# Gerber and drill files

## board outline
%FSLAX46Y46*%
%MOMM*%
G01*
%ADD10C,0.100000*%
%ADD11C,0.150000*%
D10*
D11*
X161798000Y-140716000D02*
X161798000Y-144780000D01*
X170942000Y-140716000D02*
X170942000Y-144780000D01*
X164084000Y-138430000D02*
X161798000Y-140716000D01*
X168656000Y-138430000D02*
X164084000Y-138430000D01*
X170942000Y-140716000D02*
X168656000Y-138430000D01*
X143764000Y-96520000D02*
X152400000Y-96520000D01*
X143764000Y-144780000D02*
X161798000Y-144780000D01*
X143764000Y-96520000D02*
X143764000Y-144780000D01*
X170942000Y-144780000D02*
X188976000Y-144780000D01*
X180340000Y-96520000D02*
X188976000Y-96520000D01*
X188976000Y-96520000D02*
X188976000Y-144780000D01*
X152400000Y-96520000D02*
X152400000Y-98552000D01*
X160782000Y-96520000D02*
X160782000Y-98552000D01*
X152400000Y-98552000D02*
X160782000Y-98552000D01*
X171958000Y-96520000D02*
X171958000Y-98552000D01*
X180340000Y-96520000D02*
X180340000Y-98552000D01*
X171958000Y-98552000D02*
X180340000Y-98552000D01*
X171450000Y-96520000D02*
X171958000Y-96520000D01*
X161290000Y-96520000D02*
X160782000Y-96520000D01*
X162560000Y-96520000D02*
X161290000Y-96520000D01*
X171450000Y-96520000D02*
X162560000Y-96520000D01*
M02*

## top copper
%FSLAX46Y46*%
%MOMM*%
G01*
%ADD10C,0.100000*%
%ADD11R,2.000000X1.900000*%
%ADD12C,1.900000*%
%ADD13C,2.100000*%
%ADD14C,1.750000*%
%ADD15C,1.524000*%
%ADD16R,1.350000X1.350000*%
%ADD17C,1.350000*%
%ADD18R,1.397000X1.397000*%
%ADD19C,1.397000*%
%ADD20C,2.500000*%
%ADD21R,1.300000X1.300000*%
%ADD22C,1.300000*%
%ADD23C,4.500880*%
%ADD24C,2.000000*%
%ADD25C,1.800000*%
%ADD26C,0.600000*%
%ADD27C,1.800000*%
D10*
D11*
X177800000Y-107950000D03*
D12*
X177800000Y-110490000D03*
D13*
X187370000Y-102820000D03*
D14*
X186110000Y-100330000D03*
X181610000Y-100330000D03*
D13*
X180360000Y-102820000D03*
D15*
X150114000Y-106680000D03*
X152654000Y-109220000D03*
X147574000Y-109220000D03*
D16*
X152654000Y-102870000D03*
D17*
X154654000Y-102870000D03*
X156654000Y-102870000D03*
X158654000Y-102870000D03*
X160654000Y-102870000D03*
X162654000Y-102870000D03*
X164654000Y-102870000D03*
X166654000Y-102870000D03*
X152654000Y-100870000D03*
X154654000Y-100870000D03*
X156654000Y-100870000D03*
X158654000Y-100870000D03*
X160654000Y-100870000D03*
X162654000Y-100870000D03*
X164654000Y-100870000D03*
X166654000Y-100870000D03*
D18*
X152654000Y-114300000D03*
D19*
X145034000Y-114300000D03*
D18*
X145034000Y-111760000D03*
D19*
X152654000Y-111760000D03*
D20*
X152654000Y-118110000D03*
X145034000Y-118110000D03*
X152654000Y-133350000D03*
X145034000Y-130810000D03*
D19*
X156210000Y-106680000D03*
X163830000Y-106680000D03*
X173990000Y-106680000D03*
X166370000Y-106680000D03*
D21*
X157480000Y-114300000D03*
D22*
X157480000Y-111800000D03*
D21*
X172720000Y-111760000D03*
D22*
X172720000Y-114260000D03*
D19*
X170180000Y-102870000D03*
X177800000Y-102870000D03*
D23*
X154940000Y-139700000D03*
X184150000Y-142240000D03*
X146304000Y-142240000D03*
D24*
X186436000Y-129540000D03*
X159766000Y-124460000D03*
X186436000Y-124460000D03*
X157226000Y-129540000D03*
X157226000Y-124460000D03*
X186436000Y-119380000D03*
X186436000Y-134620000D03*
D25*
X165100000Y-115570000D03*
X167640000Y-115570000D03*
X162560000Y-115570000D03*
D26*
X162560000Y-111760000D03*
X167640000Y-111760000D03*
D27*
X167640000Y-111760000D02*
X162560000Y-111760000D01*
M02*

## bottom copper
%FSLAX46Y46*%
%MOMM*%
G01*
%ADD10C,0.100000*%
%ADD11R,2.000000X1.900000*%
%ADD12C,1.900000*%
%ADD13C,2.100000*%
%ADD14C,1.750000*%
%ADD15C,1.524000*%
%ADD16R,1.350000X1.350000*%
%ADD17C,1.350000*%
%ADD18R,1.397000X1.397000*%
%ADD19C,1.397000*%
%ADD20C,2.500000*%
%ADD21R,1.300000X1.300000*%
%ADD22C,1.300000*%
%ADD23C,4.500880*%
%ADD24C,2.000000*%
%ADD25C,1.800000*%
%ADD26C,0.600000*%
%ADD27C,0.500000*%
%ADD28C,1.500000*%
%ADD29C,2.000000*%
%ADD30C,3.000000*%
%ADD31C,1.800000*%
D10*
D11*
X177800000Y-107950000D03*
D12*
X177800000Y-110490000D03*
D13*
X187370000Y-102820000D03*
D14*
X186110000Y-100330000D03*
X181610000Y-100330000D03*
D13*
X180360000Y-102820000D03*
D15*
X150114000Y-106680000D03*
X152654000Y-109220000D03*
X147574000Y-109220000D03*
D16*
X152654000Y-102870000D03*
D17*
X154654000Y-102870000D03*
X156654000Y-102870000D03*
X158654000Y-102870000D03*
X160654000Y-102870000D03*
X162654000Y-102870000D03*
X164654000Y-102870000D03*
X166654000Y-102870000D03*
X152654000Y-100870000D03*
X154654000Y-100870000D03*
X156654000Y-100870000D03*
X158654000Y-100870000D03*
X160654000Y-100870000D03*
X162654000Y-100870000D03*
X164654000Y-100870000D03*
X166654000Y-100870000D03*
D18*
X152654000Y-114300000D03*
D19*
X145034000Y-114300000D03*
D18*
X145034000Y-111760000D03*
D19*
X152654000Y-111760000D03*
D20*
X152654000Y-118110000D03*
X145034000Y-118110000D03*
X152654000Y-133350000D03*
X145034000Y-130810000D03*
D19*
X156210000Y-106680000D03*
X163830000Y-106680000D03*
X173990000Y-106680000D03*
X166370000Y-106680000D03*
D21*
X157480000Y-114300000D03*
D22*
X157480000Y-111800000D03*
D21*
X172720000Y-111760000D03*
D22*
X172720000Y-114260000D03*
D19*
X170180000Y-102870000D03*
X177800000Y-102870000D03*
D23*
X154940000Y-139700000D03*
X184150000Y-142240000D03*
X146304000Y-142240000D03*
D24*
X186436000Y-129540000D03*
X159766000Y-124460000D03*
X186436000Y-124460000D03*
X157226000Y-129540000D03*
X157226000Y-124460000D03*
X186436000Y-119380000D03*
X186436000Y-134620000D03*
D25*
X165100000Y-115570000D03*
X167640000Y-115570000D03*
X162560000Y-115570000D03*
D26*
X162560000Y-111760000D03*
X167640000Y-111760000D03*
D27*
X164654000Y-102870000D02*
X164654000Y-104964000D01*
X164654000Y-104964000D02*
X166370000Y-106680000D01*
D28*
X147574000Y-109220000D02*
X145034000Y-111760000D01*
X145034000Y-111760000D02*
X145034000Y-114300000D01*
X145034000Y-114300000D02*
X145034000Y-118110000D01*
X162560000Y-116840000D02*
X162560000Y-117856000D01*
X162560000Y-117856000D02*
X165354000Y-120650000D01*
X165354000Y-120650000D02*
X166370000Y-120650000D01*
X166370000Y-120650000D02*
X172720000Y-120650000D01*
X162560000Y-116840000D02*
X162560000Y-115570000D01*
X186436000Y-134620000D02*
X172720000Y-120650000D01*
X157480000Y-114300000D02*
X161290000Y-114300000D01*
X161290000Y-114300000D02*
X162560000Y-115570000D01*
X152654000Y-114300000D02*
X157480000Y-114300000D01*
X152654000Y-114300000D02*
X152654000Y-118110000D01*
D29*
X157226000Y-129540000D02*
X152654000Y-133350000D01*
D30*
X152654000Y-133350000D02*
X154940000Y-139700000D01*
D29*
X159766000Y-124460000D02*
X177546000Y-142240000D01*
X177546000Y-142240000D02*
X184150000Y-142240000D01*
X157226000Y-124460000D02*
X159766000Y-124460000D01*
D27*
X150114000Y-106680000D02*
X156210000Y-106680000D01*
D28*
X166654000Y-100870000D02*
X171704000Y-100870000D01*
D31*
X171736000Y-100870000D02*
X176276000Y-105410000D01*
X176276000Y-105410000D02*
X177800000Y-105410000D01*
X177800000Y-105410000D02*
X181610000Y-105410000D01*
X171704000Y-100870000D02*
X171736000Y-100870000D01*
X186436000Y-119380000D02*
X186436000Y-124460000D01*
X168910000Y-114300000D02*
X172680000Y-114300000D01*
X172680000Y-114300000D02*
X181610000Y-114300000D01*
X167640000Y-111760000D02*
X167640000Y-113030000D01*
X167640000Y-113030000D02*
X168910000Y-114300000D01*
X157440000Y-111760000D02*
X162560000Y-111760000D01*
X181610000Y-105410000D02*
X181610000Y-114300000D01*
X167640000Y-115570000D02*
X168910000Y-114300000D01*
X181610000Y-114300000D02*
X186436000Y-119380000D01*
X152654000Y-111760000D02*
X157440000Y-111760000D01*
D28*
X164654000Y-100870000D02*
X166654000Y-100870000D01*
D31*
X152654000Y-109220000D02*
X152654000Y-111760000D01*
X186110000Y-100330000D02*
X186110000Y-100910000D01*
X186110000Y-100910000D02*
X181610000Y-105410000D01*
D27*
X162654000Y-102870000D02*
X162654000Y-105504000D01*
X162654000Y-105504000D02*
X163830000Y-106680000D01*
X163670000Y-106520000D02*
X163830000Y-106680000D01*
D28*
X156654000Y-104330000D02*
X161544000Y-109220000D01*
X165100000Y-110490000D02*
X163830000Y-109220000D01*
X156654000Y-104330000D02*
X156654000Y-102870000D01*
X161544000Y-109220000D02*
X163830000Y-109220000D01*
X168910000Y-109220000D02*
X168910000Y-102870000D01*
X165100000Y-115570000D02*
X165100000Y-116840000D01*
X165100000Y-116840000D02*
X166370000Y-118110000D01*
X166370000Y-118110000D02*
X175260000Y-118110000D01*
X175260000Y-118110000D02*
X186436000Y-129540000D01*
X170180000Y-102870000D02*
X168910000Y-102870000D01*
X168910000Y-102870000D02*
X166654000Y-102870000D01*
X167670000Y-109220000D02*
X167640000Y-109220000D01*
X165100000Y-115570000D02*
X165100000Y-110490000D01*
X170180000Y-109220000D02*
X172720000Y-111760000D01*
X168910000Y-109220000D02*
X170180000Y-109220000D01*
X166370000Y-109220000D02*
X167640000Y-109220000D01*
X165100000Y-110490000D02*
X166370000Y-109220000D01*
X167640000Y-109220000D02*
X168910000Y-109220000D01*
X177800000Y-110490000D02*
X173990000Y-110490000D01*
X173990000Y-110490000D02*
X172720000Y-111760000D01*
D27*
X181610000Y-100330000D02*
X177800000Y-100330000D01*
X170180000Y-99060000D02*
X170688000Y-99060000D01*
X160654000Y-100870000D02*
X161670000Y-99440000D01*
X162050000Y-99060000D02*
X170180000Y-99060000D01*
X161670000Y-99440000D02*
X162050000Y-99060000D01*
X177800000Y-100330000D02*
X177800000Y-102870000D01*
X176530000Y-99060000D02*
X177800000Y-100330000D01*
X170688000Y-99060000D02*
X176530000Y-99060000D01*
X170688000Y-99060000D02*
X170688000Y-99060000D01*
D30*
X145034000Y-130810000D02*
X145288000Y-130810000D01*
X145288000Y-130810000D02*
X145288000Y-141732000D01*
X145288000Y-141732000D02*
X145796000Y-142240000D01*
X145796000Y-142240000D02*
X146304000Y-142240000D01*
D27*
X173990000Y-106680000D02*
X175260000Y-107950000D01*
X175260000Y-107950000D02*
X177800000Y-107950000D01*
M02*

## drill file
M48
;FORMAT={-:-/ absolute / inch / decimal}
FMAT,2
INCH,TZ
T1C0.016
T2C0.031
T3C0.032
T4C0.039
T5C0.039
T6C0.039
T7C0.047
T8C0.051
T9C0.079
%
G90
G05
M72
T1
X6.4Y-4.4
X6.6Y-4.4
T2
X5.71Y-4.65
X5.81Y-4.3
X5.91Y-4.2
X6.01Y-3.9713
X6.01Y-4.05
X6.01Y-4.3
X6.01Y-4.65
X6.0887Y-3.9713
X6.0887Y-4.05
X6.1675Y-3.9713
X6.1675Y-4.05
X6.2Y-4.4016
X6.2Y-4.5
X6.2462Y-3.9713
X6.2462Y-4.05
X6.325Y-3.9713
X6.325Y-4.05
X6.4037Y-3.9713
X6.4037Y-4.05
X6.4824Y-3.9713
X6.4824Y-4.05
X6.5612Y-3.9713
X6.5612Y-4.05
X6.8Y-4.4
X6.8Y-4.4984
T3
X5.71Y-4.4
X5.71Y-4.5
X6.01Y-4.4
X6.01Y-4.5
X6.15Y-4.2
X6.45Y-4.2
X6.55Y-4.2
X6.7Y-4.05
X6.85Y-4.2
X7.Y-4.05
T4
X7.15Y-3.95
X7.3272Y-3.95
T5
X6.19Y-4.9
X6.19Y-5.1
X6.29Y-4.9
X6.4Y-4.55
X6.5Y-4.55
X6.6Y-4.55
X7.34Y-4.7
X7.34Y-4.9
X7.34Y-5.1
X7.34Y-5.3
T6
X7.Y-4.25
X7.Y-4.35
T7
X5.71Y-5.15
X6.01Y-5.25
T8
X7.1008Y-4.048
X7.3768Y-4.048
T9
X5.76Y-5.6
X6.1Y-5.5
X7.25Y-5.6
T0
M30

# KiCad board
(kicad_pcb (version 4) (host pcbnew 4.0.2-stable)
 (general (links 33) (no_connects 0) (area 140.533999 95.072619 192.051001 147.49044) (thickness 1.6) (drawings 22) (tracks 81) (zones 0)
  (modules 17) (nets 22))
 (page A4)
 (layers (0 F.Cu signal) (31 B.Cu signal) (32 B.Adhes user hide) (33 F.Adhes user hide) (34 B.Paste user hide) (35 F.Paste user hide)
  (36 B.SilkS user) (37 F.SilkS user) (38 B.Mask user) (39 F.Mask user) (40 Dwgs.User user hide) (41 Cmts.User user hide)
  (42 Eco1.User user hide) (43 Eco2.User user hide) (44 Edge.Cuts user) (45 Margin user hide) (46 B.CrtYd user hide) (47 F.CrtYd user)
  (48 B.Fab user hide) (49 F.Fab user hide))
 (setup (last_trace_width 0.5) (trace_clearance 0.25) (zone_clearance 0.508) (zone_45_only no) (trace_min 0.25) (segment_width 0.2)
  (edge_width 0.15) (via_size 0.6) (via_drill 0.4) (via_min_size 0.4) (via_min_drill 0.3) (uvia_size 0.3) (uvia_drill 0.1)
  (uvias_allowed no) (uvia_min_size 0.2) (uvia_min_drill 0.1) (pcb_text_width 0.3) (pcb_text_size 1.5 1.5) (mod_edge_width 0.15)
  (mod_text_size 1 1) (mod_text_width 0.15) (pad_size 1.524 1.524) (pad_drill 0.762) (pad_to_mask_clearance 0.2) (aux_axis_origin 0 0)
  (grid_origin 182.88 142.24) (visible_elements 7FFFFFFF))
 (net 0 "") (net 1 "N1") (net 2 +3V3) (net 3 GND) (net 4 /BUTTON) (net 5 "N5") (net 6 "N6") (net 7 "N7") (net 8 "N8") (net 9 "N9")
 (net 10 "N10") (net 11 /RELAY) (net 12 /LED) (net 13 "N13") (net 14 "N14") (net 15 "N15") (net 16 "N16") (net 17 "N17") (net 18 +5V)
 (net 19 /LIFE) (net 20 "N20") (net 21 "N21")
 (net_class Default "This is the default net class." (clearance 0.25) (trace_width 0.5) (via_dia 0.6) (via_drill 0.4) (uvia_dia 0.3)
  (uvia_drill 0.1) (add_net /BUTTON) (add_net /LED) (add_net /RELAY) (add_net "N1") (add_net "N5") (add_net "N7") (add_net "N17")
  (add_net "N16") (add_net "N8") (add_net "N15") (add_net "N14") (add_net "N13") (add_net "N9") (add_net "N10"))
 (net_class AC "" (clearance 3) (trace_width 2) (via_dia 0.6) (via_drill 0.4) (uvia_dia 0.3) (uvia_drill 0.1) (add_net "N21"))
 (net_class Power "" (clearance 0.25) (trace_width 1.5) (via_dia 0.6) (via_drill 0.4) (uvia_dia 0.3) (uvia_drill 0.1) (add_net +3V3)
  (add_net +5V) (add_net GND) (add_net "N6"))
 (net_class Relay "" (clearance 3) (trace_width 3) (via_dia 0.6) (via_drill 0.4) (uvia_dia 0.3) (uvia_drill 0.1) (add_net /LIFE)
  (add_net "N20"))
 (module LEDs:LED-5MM (layer F.Cu) (at 177.8 107.95 270)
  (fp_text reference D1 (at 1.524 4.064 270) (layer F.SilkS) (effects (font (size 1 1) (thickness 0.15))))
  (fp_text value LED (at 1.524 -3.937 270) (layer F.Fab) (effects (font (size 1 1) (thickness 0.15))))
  (pad 1 thru_hole rect (at 0 0) (size 2 1.9) (drill 1.00076) (layers *.Cu *.Mask F.SilkS) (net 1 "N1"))
  (pad 2 thru_hole circle (at 2.54 0 270) (size 1.9 1.9) (drill 1.00076) (layers *.Cu *.Mask F.SilkS) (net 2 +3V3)))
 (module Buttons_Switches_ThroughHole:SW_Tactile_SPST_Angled (layer F.Cu) (at 181.61 100.33)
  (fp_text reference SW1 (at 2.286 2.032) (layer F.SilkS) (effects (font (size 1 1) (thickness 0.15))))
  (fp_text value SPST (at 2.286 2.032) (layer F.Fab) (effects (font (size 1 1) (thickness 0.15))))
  (pad "" thru_hole circle (at 5.76 2.49) (size 2.1 2.1) (drill 1.3) (layers *.Cu *.Mask F.SilkS))
  (pad 2 thru_hole circle (at 4.5 0) (size 1.75 1.75) (drill 0.99) (layers *.Cu *.Mask F.SilkS) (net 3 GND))
  (pad 1 thru_hole circle (at 0 0) (size 1.75 1.75) (drill 0.99) (layers *.Cu *.Mask F.SilkS) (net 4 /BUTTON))
  (pad "" thru_hole circle (at -1.25 2.49) (size 2.1 2.1) (drill 1.3) (layers *.Cu *.Mask F.SilkS)))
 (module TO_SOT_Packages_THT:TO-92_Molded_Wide (layer F.Cu) (at 147.574 109.22)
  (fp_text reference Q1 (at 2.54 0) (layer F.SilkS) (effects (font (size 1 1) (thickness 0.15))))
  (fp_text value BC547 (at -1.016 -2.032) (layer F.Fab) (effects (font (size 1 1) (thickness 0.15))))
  (pad 2 thru_hole circle (at 2.54 -2.54 90) (size 1.524 1.524) (drill 0.8) (layers *.Cu *.Mask F.SilkS) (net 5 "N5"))
  (pad 3 thru_hole circle (at 5.08 0 90) (size 1.524 1.524) (drill 0.8) (layers *.Cu *.Mask F.SilkS) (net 3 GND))
  (pad 1 thru_hole circle (at 0 0 90) (size 1.524 1.524) (drill 0.8) (layers *.Cu *.Mask F.SilkS) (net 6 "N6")))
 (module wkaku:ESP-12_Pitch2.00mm (layer F.Cu) (at 152.654 102.87 90)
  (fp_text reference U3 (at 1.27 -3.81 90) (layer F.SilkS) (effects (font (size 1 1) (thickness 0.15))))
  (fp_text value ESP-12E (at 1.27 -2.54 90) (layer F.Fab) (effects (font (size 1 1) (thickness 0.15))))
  (pad 1 thru_hole rect (at 0 0 90) (size 1.35 1.35) (drill 0.8) (layers *.Cu *.Mask) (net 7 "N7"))
  (pad 2 thru_hole circle (at 0 2 90) (size 1.35 1.35) (drill 0.8) (layers *.Cu *.Mask) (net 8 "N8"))
  (pad 3 thru_hole circle (at 0 4 90) (size 1.35 1.35) (drill 0.8) (layers *.Cu *.Mask) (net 2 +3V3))
  (pad 4 thru_hole circle (at 0 6 90) (size 1.35 1.35) (drill 0.8) (layers *.Cu *.Mask) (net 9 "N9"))
  (pad 5 thru_hole circle (at 0 8 90) (size 1.35 1.35) (drill 0.8) (layers *.Cu *.Mask) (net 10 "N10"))
  (pad 6 thru_hole circle (at 0 10 90) (size 1.35 1.35) (drill 0.8) (layers *.Cu *.Mask) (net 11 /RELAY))
  (pad 7 thru_hole circle (at 0 12 90) (size 1.35 1.35) (drill 0.8) (layers *.Cu *.Mask) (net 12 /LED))
  (pad 8 thru_hole circle (at 0 14 90) (size 1.35 1.35) (drill 0.8) (layers *.Cu *.Mask) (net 2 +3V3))
  (pad 22 thru_hole circle (at 2 0 90) (size 1.35 1.35) (drill 0.8) (layers *.Cu *.Mask) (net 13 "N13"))
  (pad 21 thru_hole circle (at 2 2 90) (size 1.35 1.35) (drill 0.8) (layers *.Cu *.Mask) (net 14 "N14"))
  (pad 20 thru_hole circle (at 2 4 90) (size 1.35 1.35) (drill 0.8) (layers *.Cu *.Mask) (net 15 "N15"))
  (pad 19 thru_hole circle (at 2 6 90) (size 1.35 1.35) (drill 0.8) (layers *.Cu *.Mask) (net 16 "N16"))
  (pad 18 thru_hole circle (at 2 8 90) (size 1.35 1.35) (drill 0.8) (layers *.Cu *.Mask) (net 4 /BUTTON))
  (pad 17 thru_hole circle (at 2 10 90) (size 1.35 1.35) (drill 0.8) (layers *.Cu *.Mask) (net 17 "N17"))
  (pad 16 thru_hole circle (at 2 12 90) (size 1.35 1.35) (drill 0.8) (layers *.Cu *.Mask) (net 3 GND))
  (pad 15 thru_hole circle (at 2 14 90) (size 1.35 1.35) (drill 0.8) (layers *.Cu *.Mask) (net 3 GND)))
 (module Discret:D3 (layer F.Cu) (at 148.844 114.3)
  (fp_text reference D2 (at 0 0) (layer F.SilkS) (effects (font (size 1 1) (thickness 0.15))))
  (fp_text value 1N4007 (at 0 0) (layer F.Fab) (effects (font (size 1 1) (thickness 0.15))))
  (pad 1 thru_hole rect (at 3.81 0) (size 1.397 1.397) (drill 0.8128) (layers *.Cu *.Mask F.SilkS) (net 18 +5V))
  (pad 2 thru_hole circle (at -3.81 0) (size 1.397 1.397) (drill 0.8128) (layers *.Cu *.Mask F.SilkS) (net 6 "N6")))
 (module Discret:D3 (layer F.Cu) (at 148.844 111.76 180)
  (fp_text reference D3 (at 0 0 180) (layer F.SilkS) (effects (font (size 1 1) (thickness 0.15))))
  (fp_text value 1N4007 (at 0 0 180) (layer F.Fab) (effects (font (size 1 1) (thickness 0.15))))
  (pad 1 thru_hole rect (at 3.81 0 180) (size 1.397 1.397) (drill 0.8128) (layers *.Cu *.Mask F.SilkS) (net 6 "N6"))
  (pad 2 thru_hole circle (at -3.81 0 180) (size 1.397 1.397) (drill 0.8128) (layers *.Cu *.Mask F.SilkS) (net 3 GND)))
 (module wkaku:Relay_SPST (layer F.Cu) (at 145.034 118.11 270)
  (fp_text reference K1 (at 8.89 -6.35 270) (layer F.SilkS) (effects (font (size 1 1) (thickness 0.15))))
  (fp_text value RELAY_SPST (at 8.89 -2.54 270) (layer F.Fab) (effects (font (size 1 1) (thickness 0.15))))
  (pad A1 thru_hole circle (at 0 -7.62 270) (size 2.5 2.5) (drill 0.8) (layers *.Cu *.Mask F.SilkS) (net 18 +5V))
  (pad A2 thru_hole circle (at 0 0 270) (size 2.5 2.5) (drill 0.8) (layers *.Cu *.Mask F.SilkS) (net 6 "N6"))
  (pad 7 thru_hole circle (at 15.24 -7.62 270) (size 2.5 2.5) (drill 1.19888) (layers *.Cu *.Mask F.SilkS) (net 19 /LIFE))
  (pad 5 thru_hole circle (at 12.7 0 270) (size 2.5 2.5) (drill 1.19888) (layers *.Cu *.Mask F.SilkS) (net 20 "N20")))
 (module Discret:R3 (layer F.Cu) (at 160.02 106.68)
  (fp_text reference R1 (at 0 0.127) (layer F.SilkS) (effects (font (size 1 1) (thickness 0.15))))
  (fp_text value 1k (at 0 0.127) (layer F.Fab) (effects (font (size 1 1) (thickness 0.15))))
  (pad 1 thru_hole circle (at -3.81 0) (size 1.397 1.397) (drill 0.8128) (layers *.Cu *.Mask F.SilkS) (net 5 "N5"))
  (pad 2 thru_hole circle (at 3.81 0) (size 1.397 1.397) (drill 0.8128) (layers *.Cu *.Mask F.SilkS) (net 11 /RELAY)))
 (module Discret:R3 (layer F.Cu) (at 170.18 106.68 180)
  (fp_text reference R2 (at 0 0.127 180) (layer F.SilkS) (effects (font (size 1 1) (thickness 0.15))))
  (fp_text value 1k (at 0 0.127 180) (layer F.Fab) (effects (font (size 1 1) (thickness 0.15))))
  (pad 1 thru_hole circle (at -3.81 0 180) (size 1.397 1.397) (drill 0.8128) (layers *.Cu *.Mask F.SilkS) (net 1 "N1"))
  (pad 2 thru_hole circle (at 3.81 0 180) (size 1.397 1.397) (drill 0.8128) (layers *.Cu *.Mask F.SilkS) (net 12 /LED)))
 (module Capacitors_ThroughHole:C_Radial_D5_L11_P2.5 (layer F.Cu) (at 157.48 114.3 90)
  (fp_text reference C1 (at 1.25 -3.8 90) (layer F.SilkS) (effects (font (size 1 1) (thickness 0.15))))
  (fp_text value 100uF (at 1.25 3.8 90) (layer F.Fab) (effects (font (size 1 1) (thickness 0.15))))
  (pad 1 thru_hole rect (at 0 0 90) (size 1.3 1.3) (drill 0.8) (layers *.Cu *.Mask F.SilkS) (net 18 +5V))
  (pad 2 thru_hole circle (at 2.5 0 90) (size 1.3 1.3) (drill 0.8) (layers *.Cu *.Mask F.SilkS) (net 3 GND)))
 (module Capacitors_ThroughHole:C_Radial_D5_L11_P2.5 (layer F.Cu) (at 172.72 111.76 270)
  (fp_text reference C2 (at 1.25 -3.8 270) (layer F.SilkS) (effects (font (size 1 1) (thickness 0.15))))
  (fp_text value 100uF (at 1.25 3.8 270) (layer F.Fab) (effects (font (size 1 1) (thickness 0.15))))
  (pad 1 thru_hole rect (at 0 0 270) (size 1.3 1.3) (drill 0.8) (layers *.Cu *.Mask F.SilkS) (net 2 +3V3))
  (pad 2 thru_hole circle (at 2.5 0 270) (size 1.3 1.3) (drill 0.8) (layers *.Cu *.Mask F.SilkS) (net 3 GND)))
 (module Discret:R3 (layer F.Cu) (at 173.99 102.87)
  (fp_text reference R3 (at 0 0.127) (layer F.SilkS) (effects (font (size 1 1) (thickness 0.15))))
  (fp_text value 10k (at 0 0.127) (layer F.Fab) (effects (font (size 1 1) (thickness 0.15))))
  (pad 1 thru_hole circle (at -3.81 0) (size 1.397 1.397) (drill 0.8128) (layers *.Cu *.Mask F.SilkS) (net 2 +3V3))
  (pad 2 thru_hole circle (at 3.81 0) (size 1.397 1.397) (drill 0.8128) (layers *.Cu *.Mask F.SilkS) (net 4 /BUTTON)))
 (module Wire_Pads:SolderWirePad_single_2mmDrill (layer F.Cu) (at 154.94 139.7)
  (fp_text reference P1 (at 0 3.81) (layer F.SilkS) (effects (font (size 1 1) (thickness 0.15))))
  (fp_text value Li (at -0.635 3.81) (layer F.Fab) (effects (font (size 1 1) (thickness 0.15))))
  (pad 1 thru_hole circle (at 0 0) (size 4.50088 4.50088) (drill 1.99898) (layers *.Cu *.Mask F.SilkS) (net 19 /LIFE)))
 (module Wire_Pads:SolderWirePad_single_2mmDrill (layer F.Cu) (at 184.15 142.24)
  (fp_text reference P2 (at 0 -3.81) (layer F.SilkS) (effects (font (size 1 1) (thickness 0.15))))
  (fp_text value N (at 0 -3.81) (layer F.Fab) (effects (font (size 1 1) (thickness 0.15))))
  (pad 1 thru_hole circle (at 0 0) (size 4.50088 4.50088) (drill 1.99898) (layers *.Cu *.Mask F.SilkS) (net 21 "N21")))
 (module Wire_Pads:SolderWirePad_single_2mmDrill (layer F.Cu) (at 146.304 142.24)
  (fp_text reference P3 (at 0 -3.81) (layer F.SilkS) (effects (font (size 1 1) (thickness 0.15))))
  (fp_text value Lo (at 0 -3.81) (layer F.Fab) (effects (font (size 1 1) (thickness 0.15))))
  (pad 1 thru_hole circle (at 0 0) (size 4.50088 4.50088) (drill 1.99898) (layers *.Cu *.Mask F.SilkS) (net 20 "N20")))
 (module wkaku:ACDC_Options (layer F.Cu) (at 157.226 129.54)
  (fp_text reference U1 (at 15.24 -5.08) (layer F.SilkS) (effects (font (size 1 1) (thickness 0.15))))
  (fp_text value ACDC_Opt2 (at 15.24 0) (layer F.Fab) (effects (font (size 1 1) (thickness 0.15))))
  (pad 4 thru_hole circle (at 29.21 0) (size 2 2) (drill 1) (layers *.Cu *.Mask F.SilkS) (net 2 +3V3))
  (pad 7 thru_hole circle (at 2.54 -5.08) (size 2 2) (drill 1) (layers *.Cu *.Mask F.SilkS) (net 21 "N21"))
  (pad 6 thru_hole circle (at 29.21 -5.08) (size 2 2) (drill 1) (layers *.Cu *.Mask F.SilkS) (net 3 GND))
  (pad 1 thru_hole circle (at 0 0) (size 2 2) (drill 1) (layers *.Cu *.Mask F.SilkS) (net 19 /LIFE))
  (pad 2 thru_hole circle (at 0 -5.08) (size 2 2) (drill 1) (layers *.Cu *.Mask F.SilkS) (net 21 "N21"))
  (pad 5 thru_hole circle (at 29.21 -10.16) (size 2 2) (drill 1) (layers *.Cu *.Mask F.SilkS) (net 3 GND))
  (pad 3 thru_hole circle (at 29.21 5.08) (size 2 2) (drill 1) (layers *.Cu *.Mask F.SilkS) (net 18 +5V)))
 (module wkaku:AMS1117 (layer F.Cu) (at 165.1 115.57)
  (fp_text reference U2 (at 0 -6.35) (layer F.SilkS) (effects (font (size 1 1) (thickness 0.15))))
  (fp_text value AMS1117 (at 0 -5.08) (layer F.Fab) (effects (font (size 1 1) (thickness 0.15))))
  (pad 2 thru_hole circle (at 0 0) (size 1.8 1.8) (drill 1) (layers *.Cu *.Mask F.SilkS) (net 2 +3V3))
  (pad 1 thru_hole circle (at 2.54 0) (size 1.8 1.8) (drill 1) (layers *.Cu *.Mask F.SilkS) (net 3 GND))
  (pad 3 thru_hole circle (at -2.54 0) (size 1.8 1.8) (drill 1) (layers *.Cu *.Mask F.SilkS) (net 18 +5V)))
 (gr_line (start 161.798 140.716) (end 161.798 144.78) (angle 90) (layer Edge.Cuts) (width 0.15))
 (gr_line (start 170.942 140.716) (end 170.942 144.78) (angle 90) (layer Edge.Cuts) (width 0.15))
 (gr_line (start 164.084 138.43) (end 161.798 140.716) (angle 90) (layer Edge.Cuts) (width 0.15))
 (gr_line (start 168.656 138.43) (end 164.084 138.43) (angle 90) (layer Edge.Cuts) (width 0.15))
 (gr_line (start 170.942 140.716) (end 168.656 138.43) (angle 90) (layer Edge.Cuts) (width 0.15))
 (gr_line (start 143.764 96.52) (end 152.4 96.52) (angle 90) (layer Edge.Cuts) (width 0.15))
 (gr_line (start 143.764 144.78) (end 161.798 144.78) (angle 90) (layer Edge.Cuts) (width 0.15))
 (gr_line (start 143.764 96.52) (end 143.764 144.78) (angle 90) (layer Edge.Cuts) (width 0.15))
 (gr_line (start 170.942 144.78) (end 188.976 144.78) (angle 90) (layer Edge.Cuts) (width 0.15))
 (gr_line (start 180.34 96.52) (end 188.976 96.52) (angle 90) (layer Edge.Cuts) (width 0.15))
 (gr_line (start 188.976 96.52) (end 188.976 144.78) (angle 90) (layer Edge.Cuts) (width 0.15))
 (gr_line (start 152.4 96.52) (end 152.4 98.552) (angle 90) (layer Edge.Cuts) (width 0.15))
 (gr_line (start 160.782 96.52) (end 160.782 98.552) (angle 90) (layer Edge.Cuts) (width 0.15))
 (gr_line (start 152.4 98.552) (end 160.782 98.552) (angle 90) (layer Edge.Cuts) (width 0.15))
 (gr_line (start 171.958 96.52) (end 171.958 98.552) (angle 90) (layer Edge.Cuts) (width 0.15))
 (gr_line (start 180.34 96.52) (end 180.34 98.552) (angle 90) (layer Edge.Cuts) (width 0.15))
 (gr_line (start 171.958 98.552) (end 180.34 98.552) (angle 90) (layer Edge.Cuts) (width 0.15))
 (gr_line (start 171.45 96.52) (end 171.958 96.52) (angle 90) (layer Edge.Cuts) (width 0.15))
 (gr_line (start 161.29 96.52) (end 160.782 96.52) (angle 90) (layer Edge.Cuts) (width 0.15))
 (gr_line (start 162.56 96.52) (end 161.29 96.52) (angle 90) (layer Edge.Cuts) (width 0.15))
 (gr_line (start 171.45 96.52) (end 162.56 96.52) (angle 90) (layer Edge.Cuts) (width 0.15))
 (segment (start 164.654 102.87) (end 164.654 104.964) (width 0.5) (layer B.Cu) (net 12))
 (segment (start 164.654 104.964) (end 166.37 106.68) (width 0.5) (layer B.Cu) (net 12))
 (segment (start 147.574 109.22) (end 145.034 111.76) (width 1.5) (layer B.Cu) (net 6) (status 10))
 (segment (start 145.034 111.76) (end 145.034 114.3) (width 1.5) (layer B.Cu) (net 6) (status 10))
 (segment (start 145.034 114.3) (end 145.034 118.11) (width 1.5) (layer B.Cu) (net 6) (status 10))
 (segment (start 162.56 116.84) (end 162.56 117.856) (width 1.5) (layer B.Cu) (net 18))
 (segment (start 162.56 117.856) (end 165.354 120.65) (width 1.5) (layer B.Cu) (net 18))
 (segment (start 165.354 120.65) (end 166.37 120.65) (width 1.5) (layer B.Cu) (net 18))
 (segment (start 166.37 120.65) (end 172.72 120.65) (width 1.5) (layer B.Cu) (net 18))
 (segment (start 162.56 116.84) (end 162.56 115.57) (width 1.5) (layer B.Cu) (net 18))
 (segment (start 186.436 134.62) (end 172.72 120.65) (width 1.5) (layer B.Cu) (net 18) (status 10))
 (segment (start 157.48 114.3) (end 161.29 114.3) (width 1.5) (layer B.Cu) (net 18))
 (segment (start 161.29 114.3) (end 162.56 115.57) (width 1.5) (layer B.Cu) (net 18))
 (segment (start 152.654 114.3) (end 157.48 114.3) (width 1.5) (layer B.Cu) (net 18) (status 10))
 (segment (start 152.654 114.3) (end 152.654 118.11) (width 1.5) (layer B.Cu) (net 18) (status 10))
 (segment (start 157.226 129.54) (end 152.654 133.35) (width 2) (layer B.Cu) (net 19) (status 10))
 (segment (start 152.654 133.35) (end 154.94 139.7) (width 3) (layer B.Cu) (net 19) (status 20))
 (segment (start 159.766 124.46) (end 177.546 142.24) (width 2) (layer B.Cu) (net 21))
 (segment (start 177.546 142.24) (end 184.15 142.24) (width 2) (layer B.Cu) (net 21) (status 20))
 (segment (start 157.226 124.46) (end 159.766 124.46) (width 2) (layer B.Cu) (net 21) (status 30))
 (segment (start 150.114 106.68) (end 156.21 106.68) (width 0.5) (layer B.Cu) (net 5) (status 10))
 (segment (start 166.654 100.87) (end 171.704 100.87) (width 1.5) (layer B.Cu) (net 3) (status 10))
 (segment (start 171.736 100.87) (end 176.276 105.41) (width 1.8) (layer B.Cu) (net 3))
 (segment (start 176.276 105.41) (end 177.8 105.41) (width 1.8) (layer B.Cu) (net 3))
 (segment (start 177.8 105.41) (end 181.61 105.41) (width 1.8) (layer B.Cu) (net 3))
 (segment (start 171.704 100.87) (end 171.736 100.87) (width 1.8) (layer B.Cu) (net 3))
 (segment (start 186.436 119.38) (end 186.436 124.46) (width 1.8) (layer B.Cu) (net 3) (status 30))
 (segment (start 168.91 114.3) (end 172.68 114.3) (width 1.8) (layer B.Cu) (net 3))
 (segment (start 172.68 114.3) (end 181.61 114.3) (width 1.8) (layer B.Cu) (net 3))
 (segment (start 167.64 111.76) (end 167.64 113.03) (width 1.8) (layer B.Cu) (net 3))
 (segment (start 167.64 113.03) (end 168.91 114.3) (width 1.8) (layer B.Cu) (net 3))
 (segment (start 157.44 111.76) (end 162.56 111.76) (width 1.8) (layer B.Cu) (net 3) (status 10))
 (via (at 162.56 111.76) (size 0.6) (drill 0.4) (layers F.Cu B.Cu) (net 3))
 (via (at 167.64 111.76) (size 0.6) (drill 0.4) (layers F.Cu B.Cu) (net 3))
 (segment (start 167.64 111.76) (end 162.56 111.76) (width 1.8) (layer F.Cu) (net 3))
 (segment (start 181.61 105.41) (end 181.61 114.3) (width 1.8) (layer B.Cu) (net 3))
 (segment (start 167.64 115.57) (end 168.91 114.3) (width 1.8) (layer B.Cu) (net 3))
 (segment (start 181.61 114.3) (end 186.436 119.38) (width 1.8) (layer B.Cu) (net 3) (status 20))
 (segment (start 152.654 111.76) (end 157.44 111.76) (width 1.8) (layer B.Cu) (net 3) (status 10))
 (segment (start 164.654 100.87) (end 166.654 100.87) (width 1.5) (layer B.Cu) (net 3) (status 30))
 (segment (start 152.654 109.22) (end 152.654 111.76) (width 1.8) (layer B.Cu) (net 3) (status 10))
 (segment (start 186.11 100.33) (end 186.11 100.91) (width 1.8) (layer B.Cu) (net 3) (status 30))
 (segment (start 186.11 100.91) (end 181.61 105.41) (width 1.8) (layer B.Cu) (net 3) (status 10))
 (segment (start 162.654 102.87) (end 162.654 105.504) (width 0.5) (layer B.Cu) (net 11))
 (segment (start 162.654 105.504) (end 163.83 106.68) (width 0.5) (layer B.Cu) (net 11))
 (segment (start 163.67 106.52) (end 163.83 106.68) (width 0.5) (layer B.Cu) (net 11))
 (segment (start 156.654 104.33) (end 161.544 109.22) (width 1.5) (layer B.Cu) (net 2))
 (segment (start 165.1 110.49) (end 163.83 109.22) (width 1.5) (layer B.Cu) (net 2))
 (segment (start 156.654 104.33) (end 156.654 102.87) (width 1.5) (layer B.Cu) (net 2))
 (segment (start 161.544 109.22) (end 163.83 109.22) (width 1.5) (layer B.Cu) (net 2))
 (segment (start 168.91 109.22) (end 168.91 102.87) (width 1.5) (layer B.Cu) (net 2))
 (segment (start 165.1 115.57) (end 165.1 116.84) (width 1.5) (layer B.Cu) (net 2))
 (segment (start 165.1 116.84) (end 166.37 118.11) (width 1.5) (layer B.Cu) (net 2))
 (segment (start 166.37 118.11) (end 175.26 118.11) (width 1.5) (layer B.Cu) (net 2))
 (segment (start 175.26 118.11) (end 186.436 129.54) (width 1.5) (layer B.Cu) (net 2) (status 20))
 (segment (start 170.18 102.87) (end 168.91 102.87) (width 1.5) (layer B.Cu) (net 2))
 (segment (start 168.91 102.87) (end 166.654 102.87) (width 1.5) (layer B.Cu) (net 2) (status 20))
 (segment (start 167.67 109.22) (end 167.64 109.22) (width 1.5) (layer B.Cu) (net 2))
 (segment (start 165.1 115.57) (end 165.1 110.49) (width 1.5) (layer B.Cu) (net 2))
 (segment (start 170.18 109.22) (end 172.72 111.76) (width 1.5) (layer B.Cu) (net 2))
 (segment (start 168.91 109.22) (end 170.18 109.22) (width 1.5) (layer B.Cu) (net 2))
 (segment (start 166.37 109.22) (end 167.64 109.22) (width 1.5) (layer B.Cu) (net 2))
 (segment (start 165.1 110.49) (end 166.37 109.22) (width 1.5) (layer B.Cu) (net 2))
 (segment (start 167.64 109.22) (end 168.91 109.22) (width 1.5) (layer B.Cu) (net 2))
 (segment (start 177.8 110.49) (end 173.99 110.49) (width 1.5) (layer B.Cu) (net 2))
 (segment (start 173.99 110.49) (end 172.72 111.76) (width 1.5) (layer B.Cu) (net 2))
 (segment (start 181.61 100.33) (end 177.8 100.33) (width 0.5) (layer B.Cu) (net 4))
 (segment (start 170.18 99.06) (end 170.688 99.06) (width 0.5) (layer B.Cu) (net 4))
 (segment (start 160.654 100.87) (end 161.67 99.44) (width 0.5) (layer B.Cu) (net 4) (status 10))
 (segment (start 162.05 99.06) (end 170.18 99.06) (width 0.5) (layer B.Cu) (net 4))
 (segment (start 161.67 99.44) (end 162.05 99.06) (width 0.5) (layer B.Cu) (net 4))
 (segment (start 177.8 100.33) (end 177.8 102.87) (width 0.5) (layer B.Cu) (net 4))
 (segment (start 176.53 99.06) (end 177.8 100.33) (width 0.5) (layer B.Cu) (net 4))
 (segment (start 170.688 99.06) (end 176.53 99.06) (width 0.5) (layer B.Cu) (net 4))
 (segment (start 170.688 99.06) (end 170.688 99.06) (width 0.5) (layer B.Cu) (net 4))
 (segment (start 145.034 130.81) (end 145.288 130.81) (width 3) (layer B.Cu) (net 20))
 (segment (start 145.288 130.81) (end 145.288 141.732) (width 3) (layer B.Cu) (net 20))
 (segment (start 145.288 141.732) (end 145.796 142.24) (width 3) (layer B.Cu) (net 20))
 (segment (start 145.796 142.24) (end 146.304 142.24) (width 3) (layer B.Cu) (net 20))
 (segment (start 173.99 106.68) (end 175.26 107.95) (width 0.5) (layer B.Cu) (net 1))
 (segment (start 175.26 107.95) (end 177.8 107.95) (width 0.5) (layer B.Cu) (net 1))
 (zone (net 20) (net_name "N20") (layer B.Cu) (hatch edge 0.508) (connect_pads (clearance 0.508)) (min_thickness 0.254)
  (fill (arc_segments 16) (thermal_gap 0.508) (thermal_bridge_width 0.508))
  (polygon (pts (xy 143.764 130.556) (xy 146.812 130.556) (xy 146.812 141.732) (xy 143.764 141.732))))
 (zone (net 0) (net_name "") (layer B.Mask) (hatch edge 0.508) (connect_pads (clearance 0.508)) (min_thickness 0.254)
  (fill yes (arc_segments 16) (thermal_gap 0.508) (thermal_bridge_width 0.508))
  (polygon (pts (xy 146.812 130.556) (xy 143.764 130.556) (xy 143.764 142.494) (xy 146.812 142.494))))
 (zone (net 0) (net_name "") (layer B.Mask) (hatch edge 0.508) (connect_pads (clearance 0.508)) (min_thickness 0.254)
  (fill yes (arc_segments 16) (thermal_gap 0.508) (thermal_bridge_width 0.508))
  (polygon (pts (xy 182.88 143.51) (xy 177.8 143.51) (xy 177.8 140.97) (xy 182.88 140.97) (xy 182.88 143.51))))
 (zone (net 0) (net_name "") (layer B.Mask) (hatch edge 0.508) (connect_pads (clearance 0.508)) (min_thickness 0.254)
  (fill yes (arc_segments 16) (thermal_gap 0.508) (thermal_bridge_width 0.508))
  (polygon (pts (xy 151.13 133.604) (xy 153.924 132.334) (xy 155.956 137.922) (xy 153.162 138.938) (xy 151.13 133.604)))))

